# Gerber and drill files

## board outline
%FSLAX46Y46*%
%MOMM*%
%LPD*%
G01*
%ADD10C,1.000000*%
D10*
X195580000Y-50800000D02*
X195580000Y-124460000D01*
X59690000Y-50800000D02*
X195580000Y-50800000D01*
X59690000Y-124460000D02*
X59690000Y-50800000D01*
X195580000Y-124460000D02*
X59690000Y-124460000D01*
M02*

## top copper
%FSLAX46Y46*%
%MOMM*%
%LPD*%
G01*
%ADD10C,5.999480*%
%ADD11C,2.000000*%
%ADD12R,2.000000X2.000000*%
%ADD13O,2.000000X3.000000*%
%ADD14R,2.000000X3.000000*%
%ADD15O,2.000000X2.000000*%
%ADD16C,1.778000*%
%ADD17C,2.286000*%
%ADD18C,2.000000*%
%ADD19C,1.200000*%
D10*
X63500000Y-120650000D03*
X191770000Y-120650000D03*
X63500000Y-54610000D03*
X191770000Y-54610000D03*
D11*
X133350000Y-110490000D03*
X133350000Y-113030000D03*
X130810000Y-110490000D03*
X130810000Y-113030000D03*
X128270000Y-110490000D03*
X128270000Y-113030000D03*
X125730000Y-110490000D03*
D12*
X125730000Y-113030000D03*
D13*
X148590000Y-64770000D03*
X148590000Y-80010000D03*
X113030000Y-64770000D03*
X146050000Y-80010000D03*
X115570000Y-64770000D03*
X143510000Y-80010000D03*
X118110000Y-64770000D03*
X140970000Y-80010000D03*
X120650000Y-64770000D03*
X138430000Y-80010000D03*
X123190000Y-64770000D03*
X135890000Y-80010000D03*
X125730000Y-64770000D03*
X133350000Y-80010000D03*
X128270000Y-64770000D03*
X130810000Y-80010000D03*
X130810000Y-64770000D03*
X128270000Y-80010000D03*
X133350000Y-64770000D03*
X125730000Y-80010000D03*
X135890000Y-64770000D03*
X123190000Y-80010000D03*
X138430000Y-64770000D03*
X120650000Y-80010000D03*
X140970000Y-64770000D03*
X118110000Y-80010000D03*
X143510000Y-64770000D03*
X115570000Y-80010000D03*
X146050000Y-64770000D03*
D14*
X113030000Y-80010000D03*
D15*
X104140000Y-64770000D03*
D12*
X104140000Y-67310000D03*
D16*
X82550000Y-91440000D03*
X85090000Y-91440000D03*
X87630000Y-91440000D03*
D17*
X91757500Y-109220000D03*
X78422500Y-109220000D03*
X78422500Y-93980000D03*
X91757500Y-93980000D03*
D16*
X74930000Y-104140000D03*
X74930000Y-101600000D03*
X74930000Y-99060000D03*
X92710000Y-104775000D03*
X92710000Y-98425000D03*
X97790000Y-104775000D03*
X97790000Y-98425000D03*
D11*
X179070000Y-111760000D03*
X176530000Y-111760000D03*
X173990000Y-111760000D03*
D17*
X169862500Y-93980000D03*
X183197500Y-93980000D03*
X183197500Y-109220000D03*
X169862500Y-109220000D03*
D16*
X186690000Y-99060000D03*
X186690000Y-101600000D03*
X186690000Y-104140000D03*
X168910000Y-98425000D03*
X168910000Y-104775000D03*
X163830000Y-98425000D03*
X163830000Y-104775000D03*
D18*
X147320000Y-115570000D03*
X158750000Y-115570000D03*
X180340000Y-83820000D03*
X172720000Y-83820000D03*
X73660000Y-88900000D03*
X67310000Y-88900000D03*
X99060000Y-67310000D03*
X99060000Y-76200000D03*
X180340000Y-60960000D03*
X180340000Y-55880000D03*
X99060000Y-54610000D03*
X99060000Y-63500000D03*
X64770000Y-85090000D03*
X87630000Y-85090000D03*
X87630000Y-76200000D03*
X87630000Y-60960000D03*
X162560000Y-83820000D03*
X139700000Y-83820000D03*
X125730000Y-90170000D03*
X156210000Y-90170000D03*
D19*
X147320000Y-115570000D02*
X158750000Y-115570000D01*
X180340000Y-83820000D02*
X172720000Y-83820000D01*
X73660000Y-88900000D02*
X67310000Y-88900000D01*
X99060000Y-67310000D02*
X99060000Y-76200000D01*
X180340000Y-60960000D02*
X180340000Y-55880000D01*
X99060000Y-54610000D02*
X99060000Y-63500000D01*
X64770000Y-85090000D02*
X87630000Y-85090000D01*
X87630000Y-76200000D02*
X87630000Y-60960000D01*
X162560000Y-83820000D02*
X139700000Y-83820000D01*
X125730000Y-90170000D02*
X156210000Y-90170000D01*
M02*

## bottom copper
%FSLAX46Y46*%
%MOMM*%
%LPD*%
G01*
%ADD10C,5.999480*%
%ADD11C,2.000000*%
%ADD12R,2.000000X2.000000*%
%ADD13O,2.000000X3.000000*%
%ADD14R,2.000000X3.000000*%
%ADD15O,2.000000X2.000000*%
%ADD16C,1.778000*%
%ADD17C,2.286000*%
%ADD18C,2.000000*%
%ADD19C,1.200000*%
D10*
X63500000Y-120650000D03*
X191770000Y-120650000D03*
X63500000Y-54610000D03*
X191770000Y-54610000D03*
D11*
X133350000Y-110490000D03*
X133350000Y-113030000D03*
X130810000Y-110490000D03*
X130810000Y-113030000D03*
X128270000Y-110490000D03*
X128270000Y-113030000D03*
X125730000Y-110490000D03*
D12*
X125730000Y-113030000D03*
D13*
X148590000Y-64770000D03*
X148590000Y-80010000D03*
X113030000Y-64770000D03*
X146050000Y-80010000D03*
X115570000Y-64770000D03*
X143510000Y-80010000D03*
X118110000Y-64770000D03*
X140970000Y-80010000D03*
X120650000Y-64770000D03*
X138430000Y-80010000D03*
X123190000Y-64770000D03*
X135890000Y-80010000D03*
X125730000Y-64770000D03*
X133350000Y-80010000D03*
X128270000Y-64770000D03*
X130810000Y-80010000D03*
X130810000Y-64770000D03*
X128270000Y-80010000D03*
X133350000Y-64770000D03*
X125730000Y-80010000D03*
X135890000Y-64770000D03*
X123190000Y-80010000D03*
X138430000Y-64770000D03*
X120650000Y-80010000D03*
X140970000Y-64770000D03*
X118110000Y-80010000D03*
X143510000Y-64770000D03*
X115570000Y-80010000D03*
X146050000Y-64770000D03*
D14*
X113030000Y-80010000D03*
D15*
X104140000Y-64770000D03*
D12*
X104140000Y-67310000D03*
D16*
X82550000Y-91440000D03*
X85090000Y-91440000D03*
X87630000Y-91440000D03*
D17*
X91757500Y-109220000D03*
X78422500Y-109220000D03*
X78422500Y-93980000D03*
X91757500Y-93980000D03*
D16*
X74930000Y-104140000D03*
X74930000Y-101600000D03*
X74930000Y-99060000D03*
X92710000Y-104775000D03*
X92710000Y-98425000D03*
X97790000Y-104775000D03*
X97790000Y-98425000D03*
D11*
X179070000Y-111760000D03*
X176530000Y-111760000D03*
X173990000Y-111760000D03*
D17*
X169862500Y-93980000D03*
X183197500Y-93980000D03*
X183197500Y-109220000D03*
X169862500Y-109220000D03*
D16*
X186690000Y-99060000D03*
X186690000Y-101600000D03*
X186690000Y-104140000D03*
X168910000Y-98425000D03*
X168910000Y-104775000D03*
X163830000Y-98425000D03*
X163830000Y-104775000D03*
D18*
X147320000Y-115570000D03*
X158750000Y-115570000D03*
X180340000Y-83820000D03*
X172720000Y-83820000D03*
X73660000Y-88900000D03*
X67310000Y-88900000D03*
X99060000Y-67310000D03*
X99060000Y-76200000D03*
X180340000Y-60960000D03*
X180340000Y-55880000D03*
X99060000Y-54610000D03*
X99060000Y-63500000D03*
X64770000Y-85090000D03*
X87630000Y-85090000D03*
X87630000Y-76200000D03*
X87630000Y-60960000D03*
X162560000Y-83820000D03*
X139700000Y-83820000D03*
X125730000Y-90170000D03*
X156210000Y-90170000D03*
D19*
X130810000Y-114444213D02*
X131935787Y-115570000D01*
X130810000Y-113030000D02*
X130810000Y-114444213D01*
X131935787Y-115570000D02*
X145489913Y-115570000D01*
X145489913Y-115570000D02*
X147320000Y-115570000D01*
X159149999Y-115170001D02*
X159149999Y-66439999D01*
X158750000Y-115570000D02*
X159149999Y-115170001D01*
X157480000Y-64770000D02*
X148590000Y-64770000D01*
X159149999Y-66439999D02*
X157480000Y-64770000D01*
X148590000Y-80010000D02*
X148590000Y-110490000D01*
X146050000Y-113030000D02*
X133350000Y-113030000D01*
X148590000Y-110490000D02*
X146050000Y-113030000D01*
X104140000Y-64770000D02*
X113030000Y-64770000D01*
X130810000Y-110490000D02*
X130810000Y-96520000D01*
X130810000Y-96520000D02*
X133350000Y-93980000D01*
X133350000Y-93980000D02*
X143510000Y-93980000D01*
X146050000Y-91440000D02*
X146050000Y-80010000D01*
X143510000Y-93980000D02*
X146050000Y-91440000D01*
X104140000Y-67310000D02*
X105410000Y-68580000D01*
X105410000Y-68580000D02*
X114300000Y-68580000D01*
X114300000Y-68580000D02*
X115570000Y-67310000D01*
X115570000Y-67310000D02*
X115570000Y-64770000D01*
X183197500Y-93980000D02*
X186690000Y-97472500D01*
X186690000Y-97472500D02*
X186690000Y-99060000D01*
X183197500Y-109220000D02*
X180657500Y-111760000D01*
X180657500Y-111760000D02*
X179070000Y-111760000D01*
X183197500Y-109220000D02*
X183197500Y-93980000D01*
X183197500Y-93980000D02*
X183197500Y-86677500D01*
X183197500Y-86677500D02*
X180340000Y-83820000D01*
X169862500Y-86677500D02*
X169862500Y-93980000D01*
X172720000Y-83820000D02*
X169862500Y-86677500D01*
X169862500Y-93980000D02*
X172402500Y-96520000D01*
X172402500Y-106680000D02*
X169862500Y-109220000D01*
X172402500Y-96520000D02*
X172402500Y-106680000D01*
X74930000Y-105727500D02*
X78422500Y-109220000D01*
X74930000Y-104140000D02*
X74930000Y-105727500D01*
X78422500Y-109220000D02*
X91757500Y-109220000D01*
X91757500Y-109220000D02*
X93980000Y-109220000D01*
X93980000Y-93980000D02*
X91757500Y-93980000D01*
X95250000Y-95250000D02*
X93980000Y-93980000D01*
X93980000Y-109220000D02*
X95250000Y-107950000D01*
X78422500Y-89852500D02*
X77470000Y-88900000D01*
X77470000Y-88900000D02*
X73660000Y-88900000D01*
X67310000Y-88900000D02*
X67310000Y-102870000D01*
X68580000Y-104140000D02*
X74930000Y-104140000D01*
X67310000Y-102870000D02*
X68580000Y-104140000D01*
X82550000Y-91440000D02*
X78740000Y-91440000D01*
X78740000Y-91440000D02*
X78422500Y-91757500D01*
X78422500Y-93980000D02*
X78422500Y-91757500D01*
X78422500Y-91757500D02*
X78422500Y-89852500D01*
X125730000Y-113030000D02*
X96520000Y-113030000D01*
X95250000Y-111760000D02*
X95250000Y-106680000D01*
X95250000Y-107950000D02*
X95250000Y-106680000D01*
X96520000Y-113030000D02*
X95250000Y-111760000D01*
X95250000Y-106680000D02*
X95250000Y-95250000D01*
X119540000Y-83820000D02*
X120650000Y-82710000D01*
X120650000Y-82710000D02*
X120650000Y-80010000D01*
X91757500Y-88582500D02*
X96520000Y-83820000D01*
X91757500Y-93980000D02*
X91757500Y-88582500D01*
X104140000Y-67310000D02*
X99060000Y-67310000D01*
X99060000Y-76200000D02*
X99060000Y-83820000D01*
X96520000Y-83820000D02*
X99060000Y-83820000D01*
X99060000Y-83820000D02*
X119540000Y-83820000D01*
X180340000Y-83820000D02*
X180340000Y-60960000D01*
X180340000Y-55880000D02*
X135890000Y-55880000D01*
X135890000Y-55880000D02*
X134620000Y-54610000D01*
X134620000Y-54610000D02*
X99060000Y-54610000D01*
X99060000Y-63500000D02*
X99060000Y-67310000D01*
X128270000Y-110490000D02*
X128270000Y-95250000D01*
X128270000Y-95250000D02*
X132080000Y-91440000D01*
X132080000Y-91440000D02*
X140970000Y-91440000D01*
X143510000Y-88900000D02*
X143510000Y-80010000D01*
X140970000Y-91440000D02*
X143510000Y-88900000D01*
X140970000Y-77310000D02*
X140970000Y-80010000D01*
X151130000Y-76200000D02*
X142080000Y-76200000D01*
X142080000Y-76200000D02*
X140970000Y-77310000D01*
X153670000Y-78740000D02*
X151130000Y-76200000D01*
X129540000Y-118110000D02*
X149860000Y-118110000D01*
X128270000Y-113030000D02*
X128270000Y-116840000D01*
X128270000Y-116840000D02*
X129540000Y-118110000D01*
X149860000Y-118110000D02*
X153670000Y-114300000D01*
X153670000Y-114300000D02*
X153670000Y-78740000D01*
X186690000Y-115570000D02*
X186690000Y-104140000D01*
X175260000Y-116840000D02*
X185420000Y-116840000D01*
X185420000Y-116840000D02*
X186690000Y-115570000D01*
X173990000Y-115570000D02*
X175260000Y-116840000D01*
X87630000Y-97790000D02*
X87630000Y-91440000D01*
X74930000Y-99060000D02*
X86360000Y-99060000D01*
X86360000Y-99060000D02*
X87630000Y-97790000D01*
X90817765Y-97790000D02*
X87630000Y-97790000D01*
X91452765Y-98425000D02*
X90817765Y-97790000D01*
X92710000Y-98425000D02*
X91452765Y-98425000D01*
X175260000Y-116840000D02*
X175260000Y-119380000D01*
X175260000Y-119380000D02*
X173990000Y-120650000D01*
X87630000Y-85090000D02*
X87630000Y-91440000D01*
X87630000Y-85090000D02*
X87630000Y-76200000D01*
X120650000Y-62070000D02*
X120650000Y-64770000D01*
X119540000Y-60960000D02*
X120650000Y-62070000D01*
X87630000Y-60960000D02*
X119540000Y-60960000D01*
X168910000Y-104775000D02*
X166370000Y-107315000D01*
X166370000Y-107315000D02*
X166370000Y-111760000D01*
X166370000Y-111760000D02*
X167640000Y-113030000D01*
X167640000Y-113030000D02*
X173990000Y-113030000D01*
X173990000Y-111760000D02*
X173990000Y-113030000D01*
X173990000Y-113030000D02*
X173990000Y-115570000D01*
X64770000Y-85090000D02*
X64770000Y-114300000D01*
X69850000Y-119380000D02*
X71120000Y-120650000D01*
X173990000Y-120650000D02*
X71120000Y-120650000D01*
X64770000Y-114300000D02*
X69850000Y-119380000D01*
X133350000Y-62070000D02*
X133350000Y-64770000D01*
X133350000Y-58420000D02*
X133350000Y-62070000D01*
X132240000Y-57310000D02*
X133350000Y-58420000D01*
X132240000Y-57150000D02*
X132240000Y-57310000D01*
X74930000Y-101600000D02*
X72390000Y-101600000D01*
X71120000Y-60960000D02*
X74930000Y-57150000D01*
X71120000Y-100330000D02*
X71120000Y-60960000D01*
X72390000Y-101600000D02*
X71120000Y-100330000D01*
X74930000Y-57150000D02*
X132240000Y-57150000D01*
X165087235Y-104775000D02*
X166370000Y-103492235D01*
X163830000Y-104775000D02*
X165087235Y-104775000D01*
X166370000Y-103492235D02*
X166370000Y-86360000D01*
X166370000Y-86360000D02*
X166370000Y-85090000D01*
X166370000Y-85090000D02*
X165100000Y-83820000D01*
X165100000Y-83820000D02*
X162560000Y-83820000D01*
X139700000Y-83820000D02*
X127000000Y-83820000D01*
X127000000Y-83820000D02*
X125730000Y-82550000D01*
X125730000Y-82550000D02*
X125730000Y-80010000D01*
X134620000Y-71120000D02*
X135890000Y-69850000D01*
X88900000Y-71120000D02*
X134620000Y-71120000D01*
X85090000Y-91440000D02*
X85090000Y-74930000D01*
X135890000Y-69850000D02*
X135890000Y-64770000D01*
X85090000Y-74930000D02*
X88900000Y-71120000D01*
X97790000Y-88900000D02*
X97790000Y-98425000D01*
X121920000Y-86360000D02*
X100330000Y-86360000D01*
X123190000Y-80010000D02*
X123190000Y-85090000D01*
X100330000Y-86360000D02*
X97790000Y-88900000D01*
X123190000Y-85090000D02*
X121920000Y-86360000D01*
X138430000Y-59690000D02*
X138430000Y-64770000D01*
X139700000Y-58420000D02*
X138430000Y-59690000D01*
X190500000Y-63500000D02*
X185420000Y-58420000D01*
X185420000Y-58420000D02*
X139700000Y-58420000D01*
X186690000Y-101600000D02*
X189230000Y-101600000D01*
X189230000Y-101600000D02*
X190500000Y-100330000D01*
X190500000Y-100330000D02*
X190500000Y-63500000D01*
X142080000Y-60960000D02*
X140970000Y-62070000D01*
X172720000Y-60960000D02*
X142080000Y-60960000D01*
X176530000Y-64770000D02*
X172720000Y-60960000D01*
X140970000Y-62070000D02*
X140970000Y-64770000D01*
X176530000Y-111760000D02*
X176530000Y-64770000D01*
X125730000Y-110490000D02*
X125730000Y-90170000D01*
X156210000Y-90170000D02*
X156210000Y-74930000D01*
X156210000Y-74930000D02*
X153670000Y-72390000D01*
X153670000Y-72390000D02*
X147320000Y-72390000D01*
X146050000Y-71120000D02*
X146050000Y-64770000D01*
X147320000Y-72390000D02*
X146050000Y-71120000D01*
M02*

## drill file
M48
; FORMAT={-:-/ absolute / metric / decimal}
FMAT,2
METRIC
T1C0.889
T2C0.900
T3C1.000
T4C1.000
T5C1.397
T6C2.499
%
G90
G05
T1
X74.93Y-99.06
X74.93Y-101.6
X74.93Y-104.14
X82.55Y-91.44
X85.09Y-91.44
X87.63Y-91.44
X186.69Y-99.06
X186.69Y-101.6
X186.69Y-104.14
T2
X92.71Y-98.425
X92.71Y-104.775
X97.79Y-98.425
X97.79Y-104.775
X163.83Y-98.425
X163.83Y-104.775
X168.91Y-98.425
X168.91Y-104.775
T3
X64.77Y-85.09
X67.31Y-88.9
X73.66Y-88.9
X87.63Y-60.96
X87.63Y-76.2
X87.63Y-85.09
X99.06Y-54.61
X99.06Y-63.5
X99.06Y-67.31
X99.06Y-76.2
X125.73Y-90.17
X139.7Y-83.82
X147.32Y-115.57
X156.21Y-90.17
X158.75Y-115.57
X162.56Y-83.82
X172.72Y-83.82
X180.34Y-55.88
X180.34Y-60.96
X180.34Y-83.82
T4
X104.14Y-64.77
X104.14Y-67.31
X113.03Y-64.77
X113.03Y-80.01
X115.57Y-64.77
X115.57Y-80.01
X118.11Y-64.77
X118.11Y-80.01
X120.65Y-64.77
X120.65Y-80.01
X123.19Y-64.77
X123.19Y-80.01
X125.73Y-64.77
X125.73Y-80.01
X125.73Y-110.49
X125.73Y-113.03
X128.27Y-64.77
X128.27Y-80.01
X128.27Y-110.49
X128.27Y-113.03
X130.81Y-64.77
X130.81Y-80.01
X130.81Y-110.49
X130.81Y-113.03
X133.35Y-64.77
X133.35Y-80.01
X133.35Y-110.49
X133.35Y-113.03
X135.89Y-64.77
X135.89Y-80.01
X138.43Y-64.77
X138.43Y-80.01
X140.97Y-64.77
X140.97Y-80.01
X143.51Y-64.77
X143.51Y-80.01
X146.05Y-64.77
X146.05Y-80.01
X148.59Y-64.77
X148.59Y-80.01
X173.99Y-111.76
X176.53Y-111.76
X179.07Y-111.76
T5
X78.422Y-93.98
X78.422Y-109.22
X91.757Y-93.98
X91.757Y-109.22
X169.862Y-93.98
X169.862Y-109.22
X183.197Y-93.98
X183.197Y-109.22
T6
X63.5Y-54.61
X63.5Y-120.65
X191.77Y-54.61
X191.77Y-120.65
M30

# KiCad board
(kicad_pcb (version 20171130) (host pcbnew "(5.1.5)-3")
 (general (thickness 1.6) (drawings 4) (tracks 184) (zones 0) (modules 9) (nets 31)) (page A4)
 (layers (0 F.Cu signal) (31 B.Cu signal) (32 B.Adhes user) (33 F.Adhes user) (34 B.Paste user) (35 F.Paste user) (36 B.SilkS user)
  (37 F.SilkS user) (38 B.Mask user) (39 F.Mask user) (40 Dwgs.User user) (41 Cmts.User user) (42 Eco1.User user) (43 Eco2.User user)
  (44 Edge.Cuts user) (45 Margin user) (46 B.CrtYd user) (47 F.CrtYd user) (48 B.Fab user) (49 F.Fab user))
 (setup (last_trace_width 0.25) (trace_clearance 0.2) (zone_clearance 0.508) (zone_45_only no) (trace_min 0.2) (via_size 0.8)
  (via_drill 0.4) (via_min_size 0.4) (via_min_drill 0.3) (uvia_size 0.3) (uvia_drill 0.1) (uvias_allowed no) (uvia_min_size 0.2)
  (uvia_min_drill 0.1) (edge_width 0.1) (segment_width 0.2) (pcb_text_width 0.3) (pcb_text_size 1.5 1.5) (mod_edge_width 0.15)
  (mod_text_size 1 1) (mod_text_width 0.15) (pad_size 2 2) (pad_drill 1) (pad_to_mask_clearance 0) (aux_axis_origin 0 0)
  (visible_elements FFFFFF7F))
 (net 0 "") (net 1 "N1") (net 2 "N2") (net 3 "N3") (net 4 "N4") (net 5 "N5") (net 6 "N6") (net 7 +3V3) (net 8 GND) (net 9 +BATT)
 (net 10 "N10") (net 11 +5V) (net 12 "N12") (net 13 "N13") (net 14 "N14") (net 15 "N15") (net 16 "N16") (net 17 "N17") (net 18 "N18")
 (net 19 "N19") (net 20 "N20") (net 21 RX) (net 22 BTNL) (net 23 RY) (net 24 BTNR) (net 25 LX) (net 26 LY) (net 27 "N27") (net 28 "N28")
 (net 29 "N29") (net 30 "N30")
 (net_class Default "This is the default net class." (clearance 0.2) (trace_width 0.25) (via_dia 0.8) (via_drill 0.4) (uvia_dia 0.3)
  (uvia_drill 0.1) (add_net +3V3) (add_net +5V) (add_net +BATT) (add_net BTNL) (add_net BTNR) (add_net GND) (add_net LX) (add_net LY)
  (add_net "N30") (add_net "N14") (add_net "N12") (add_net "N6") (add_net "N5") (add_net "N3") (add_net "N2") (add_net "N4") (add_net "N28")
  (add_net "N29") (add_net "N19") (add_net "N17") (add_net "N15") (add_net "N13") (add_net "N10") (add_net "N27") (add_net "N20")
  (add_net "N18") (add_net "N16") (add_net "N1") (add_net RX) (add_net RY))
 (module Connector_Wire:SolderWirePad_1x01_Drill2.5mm (layer F.Cu) (at 63.5 120.65)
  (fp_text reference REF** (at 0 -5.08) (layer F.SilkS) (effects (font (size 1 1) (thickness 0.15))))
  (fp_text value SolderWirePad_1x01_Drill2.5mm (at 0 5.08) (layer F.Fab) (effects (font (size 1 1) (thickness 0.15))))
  (pad 1 thru_hole circle (at 0 0) (size 5.99948 5.99948) (drill 2.49936) (layers *.Cu *.Mask)))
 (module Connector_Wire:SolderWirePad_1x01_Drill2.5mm (layer F.Cu) (at 191.77 120.65)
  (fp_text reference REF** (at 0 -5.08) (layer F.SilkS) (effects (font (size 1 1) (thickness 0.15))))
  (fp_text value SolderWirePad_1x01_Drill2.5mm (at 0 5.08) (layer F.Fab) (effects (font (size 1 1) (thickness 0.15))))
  (pad 1 thru_hole circle (at 0 0) (size 5.99948 5.99948) (drill 2.49936) (layers *.Cu *.Mask)))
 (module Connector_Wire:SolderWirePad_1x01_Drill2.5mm (layer F.Cu) (at 63.5 54.61)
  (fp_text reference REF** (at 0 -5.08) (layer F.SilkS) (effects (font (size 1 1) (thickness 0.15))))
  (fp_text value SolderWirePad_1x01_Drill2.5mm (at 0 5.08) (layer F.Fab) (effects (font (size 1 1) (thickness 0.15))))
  (pad 1 thru_hole circle (at 0 0) (size 5.99948 5.99948) (drill 2.49936) (layers *.Cu *.Mask)))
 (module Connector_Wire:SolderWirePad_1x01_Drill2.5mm (layer F.Cu) (at 191.77 54.61)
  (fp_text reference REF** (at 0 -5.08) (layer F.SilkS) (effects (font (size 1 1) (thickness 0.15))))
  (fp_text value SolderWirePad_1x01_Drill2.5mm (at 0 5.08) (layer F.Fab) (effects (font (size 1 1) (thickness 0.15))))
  (pad 1 thru_hole circle (at 0 0) (size 5.99948 5.99948) (drill 2.49936) (layers *.Cu *.Mask)))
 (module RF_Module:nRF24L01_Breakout (layer F.Cu) (at 125.73 113.03 90)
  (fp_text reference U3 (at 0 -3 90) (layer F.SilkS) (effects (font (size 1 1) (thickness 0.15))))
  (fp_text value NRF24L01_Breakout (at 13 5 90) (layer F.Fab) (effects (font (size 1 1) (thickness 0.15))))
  (pad 8 thru_hole circle (at 2.54 7.62 90) (size 2 2) (drill 1) (layers *.Cu *.Mask) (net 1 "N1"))
  (pad 7 thru_hole circle (at 0 7.62 90) (size 2 2) (drill 1) (layers *.Cu *.Mask) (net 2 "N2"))
  (pad 6 thru_hole circle (at 2.54 5.08 90) (size 2 2) (drill 1) (layers *.Cu *.Mask) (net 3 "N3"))
  (pad 5 thru_hole circle (at 0 5.08 90) (size 2 2) (drill 1) (layers *.Cu *.Mask) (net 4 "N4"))
  (pad 4 thru_hole circle (at 2.54 2.54 90) (size 2 2) (drill 1) (layers *.Cu *.Mask) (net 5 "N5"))
  (pad 3 thru_hole circle (at 0 2.54 90) (size 2 2) (drill 1) (layers *.Cu *.Mask) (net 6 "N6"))
  (pad 2 thru_hole circle (at 2.54 0 90) (size 2 2) (drill 1) (layers *.Cu *.Mask) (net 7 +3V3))
  (pad 1 thru_hole rect (at 0 0 90) (size 2 2) (drill 1) (layers *.Cu *.Mask) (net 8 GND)))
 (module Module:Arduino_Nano (layer F.Cu) (at 113.03 80.01 90)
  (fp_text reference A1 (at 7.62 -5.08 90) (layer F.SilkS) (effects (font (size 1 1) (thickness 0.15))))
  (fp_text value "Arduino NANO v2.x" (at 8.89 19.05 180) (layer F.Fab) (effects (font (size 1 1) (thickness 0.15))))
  (pad 16 thru_hole oval (at 15.24 35.56 90) (size 3 2) (drill 1) (layers *.Cu *.Mask) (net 4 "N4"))
  (pad 15 thru_hole oval (at 0 35.56 90) (size 3 2) (drill 1) (layers *.Cu *.Mask) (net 2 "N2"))
  (pad 30 thru_hole oval (at 15.24 0 90) (size 3 2) (drill 1) (layers *.Cu *.Mask) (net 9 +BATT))
  (pad 14 thru_hole oval (at 0 33.02 90) (size 3 2) (drill 1) (layers *.Cu *.Mask) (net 3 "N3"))
  (pad 29 thru_hole oval (at 15.24 2.54 90) (size 3 2) (drill 1) (layers *.Cu *.Mask) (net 8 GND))
  (pad 13 thru_hole oval (at 0 30.48 90) (size 3 2) (drill 1) (layers *.Cu *.Mask) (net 5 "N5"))
  (pad 28 thru_hole oval (at 15.24 5.08 90) (size 3 2) (drill 1) (layers *.Cu *.Mask) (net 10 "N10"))
  (pad 12 thru_hole oval (at 0 27.94 90) (size 3 2) (drill 1) (layers *.Cu *.Mask) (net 6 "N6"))
  (pad 27 thru_hole oval (at 15.24 7.62 90) (size 3 2) (drill 1) (layers *.Cu *.Mask) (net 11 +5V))
  (pad 11 thru_hole oval (at 0 25.4 90) (size 3 2) (drill 1) (layers *.Cu *.Mask) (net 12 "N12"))
  (pad 26 thru_hole oval (at 15.24 10.16 90) (size 3 2) (drill 1) (layers *.Cu *.Mask) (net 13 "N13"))
  (pad 10 thru_hole oval (at 0 22.86 90) (size 3 2) (drill 1) (layers *.Cu *.Mask) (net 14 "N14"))
  (pad 25 thru_hole oval (at 15.24 12.7 90) (size 3 2) (drill 1) (layers *.Cu *.Mask) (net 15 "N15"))
  (pad 9 thru_hole oval (at 0 20.32 90) (size 3 2) (drill 1) (layers *.Cu *.Mask) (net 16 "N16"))
  (pad 24 thru_hole oval (at 15.24 15.24 90) (size 3 2) (drill 1) (layers *.Cu *.Mask) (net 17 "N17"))
  (pad 8 thru_hole oval (at 0 17.78 90) (size 3 2) (drill 1) (layers *.Cu *.Mask) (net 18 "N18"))
  (pad 23 thru_hole oval (at 15.24 17.78 90) (size 3 2) (drill 1) (layers *.Cu *.Mask) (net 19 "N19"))
  (pad 7 thru_hole oval (at 0 15.24 90) (size 3 2) (drill 1) (layers *.Cu *.Mask) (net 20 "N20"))
  (pad 22 thru_hole oval (at 15.24 20.32 90) (size 3 2) (drill 1) (layers *.Cu *.Mask) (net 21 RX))
  (pad 6 thru_hole oval (at 0 12.7 90) (size 3 2) (drill 1) (layers *.Cu *.Mask) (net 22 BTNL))
  (pad 21 thru_hole oval (at 15.24 22.86 90) (size 3 2) (drill 1) (layers *.Cu *.Mask) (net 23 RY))
  (pad 5 thru_hole oval (at 0 10.16 90) (size 3 2) (drill 1) (layers *.Cu *.Mask) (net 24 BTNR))
  (pad 20 thru_hole oval (at 15.24 25.4 90) (size 3 2) (drill 1) (layers *.Cu *.Mask) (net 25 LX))
  (pad 4 thru_hole oval (at 0 7.62 90) (size 3 2) (drill 1) (layers *.Cu *.Mask) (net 8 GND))
  (pad 19 thru_hole oval (at 15.24 27.94 90) (size 3 2) (drill 1) (layers *.Cu *.Mask) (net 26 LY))
  (pad 3 thru_hole oval (at 0 5.08 90) (size 3 2) (drill 1) (layers *.Cu *.Mask) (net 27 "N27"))
  (pad 18 thru_hole oval (at 15.24 30.48 90) (size 3 2) (drill 1) (layers *.Cu *.Mask) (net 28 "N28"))
  (pad 2 thru_hole oval (at 0 2.54 90) (size 3 2) (drill 1) (layers *.Cu *.Mask) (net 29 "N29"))
  (pad 17 thru_hole oval (at 15.24 33.02 90) (size 3 2) (drill 1) (layers *.Cu *.Mask) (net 7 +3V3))
  (pad 1 thru_hole rect (at 0 0 90) (size 3 2) (drill 1) (layers *.Cu *.Mask) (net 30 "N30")))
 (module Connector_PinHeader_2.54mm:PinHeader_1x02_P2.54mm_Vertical (layer F.Cu) (at 104.14 67.31 180)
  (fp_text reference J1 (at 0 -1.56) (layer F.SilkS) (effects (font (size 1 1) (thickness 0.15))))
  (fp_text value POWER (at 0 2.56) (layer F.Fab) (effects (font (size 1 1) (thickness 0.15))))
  (pad 2 thru_hole oval (at 0 2.54 180) (size 2 2) (drill 1) (layers *.Cu *.Mask) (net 9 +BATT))
  (pad 1 thru_hole rect (at 0 0 180) (size 2 2) (drill 1) (layers *.Cu *.Mask) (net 8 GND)))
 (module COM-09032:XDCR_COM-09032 (layer F.Cu) (at 85.09 101.6 270)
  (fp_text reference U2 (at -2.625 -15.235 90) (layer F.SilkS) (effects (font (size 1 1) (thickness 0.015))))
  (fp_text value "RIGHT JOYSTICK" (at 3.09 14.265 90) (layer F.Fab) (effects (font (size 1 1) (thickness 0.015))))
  (pad V3 thru_hole circle (at -10.16 2.54 270) (size 1.778 1.778) (drill 0.889) (layers *.Cu *.Mask) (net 8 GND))
  (pad V2 thru_hole circle (at -10.16 0 270) (size 1.778 1.778) (drill 0.889) (layers *.Cu *.Mask) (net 23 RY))
  (pad V1 thru_hole circle (at -10.16 -2.54 270) (size 1.778 1.778) (drill 0.889) (layers *.Cu *.Mask) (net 11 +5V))
  (pad S4 thru_hole circle (at 7.62 -6.6675 270) (size 2.286 2.286) (drill 1.397) (layers *.Cu *.Mask) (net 8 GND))
  (pad S3 thru_hole circle (at 7.62 6.6675 270) (size 2.286 2.286) (drill 1.397) (layers *.Cu *.Mask) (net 8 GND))
  (pad S2 thru_hole circle (at -7.62 6.6675 270) (size 2.286 2.286) (drill 1.397) (layers *.Cu *.Mask) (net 8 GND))
  (pad S1 thru_hole circle (at -7.62 -6.6675 270) (size 2.286 2.286) (drill 1.397) (layers *.Cu *.Mask) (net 8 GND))
  (pad H3 thru_hole circle (at 2.54 10.16 270) (size 1.778 1.778) (drill 0.889) (layers *.Cu *.Mask) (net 8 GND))
  (pad H2 thru_hole circle (at 0 10.16 270) (size 1.778 1.778) (drill 0.889) (layers *.Cu *.Mask) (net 21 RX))
  (pad H1 thru_hole circle (at -2.54 10.16 270) (size 1.778 1.778) (drill 0.889) (layers *.Cu *.Mask) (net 11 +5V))
  (pad B2B thru_hole circle (at 3.175 -7.62 270) (size 1.778 1.778) (drill 0.9) (layers *.Cu *.Mask))
  (pad B2A thru_hole circle (at -3.175 -7.62 270) (size 1.778 1.778) (drill 0.9) (layers *.Cu *.Mask) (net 11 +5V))
  (pad B1B thru_hole circle (at 3.175 -12.7 270) (size 1.778 1.778) (drill 0.9) (layers *.Cu *.Mask))
  (pad B1A thru_hole circle (at -3.175 -12.7 270) (size 1.778 1.778) (drill 0.9) (layers *.Cu *.Mask) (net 24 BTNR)))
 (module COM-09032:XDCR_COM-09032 (layer F.Cu) (at 176.53 101.6 90)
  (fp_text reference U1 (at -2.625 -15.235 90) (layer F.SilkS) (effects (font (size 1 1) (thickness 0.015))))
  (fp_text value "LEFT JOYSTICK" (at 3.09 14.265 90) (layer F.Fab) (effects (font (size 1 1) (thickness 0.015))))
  (pad V3 thru_hole circle (at -10.16 2.54 90) (size 2 2) (drill 1) (layers *.Cu *.Mask) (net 8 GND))
  (pad V2 thru_hole circle (at -10.16 0 90) (size 2 2) (drill 1) (layers *.Cu *.Mask) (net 26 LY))
  (pad V1 thru_hole circle (at -10.16 -2.54 90) (size 2 2) (drill 1) (layers *.Cu *.Mask) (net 11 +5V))
  (pad S4 thru_hole circle (at 7.62 -6.6675 90) (size 2.286 2.286) (drill 1.397) (layers *.Cu *.Mask) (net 8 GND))
  (pad S3 thru_hole circle (at 7.62 6.6675 90) (size 2.286 2.286) (drill 1.397) (layers *.Cu *.Mask) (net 8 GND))
  (pad S2 thru_hole circle (at -7.62 6.6675 90) (size 2.286 2.286) (drill 1.397) (layers *.Cu *.Mask) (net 8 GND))
  (pad S1 thru_hole circle (at -7.62 -6.6675 90) (size 2.286 2.286) (drill 1.397) (layers *.Cu *.Mask) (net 8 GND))
  (pad H3 thru_hole circle (at 2.54 10.16 90) (size 1.778 1.778) (drill 0.889) (layers *.Cu *.Mask) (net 8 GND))
  (pad H2 thru_hole circle (at 0 10.16 90) (size 1.778 1.778) (drill 0.889) (layers *.Cu *.Mask) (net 25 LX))
  (pad H1 thru_hole circle (at -2.54 10.16 90) (size 1.778 1.778) (drill 0.889) (layers *.Cu *.Mask) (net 11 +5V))
  (pad B2B thru_hole circle (at 3.175 -7.62 90) (size 1.778 1.778) (drill 0.9) (layers *.Cu *.Mask))
  (pad B2A thru_hole circle (at -3.175 -7.62 90) (size 1.778 1.778) (drill 0.9) (layers *.Cu *.Mask) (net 11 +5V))
  (pad B1B thru_hole circle (at 3.175 -12.7 90) (size 1.778 1.778) (drill 0.9) (layers *.Cu *.Mask))
  (pad B1A thru_hole circle (at -3.175 -12.7 90) (size 1.778 1.778) (drill 0.9) (layers *.Cu *.Mask) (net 22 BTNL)))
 (gr_line (start 195.58 50.8) (end 195.58 124.46) (layer Edge.Cuts) (width 1))
 (gr_line (start 59.69 50.8) (end 195.58 50.8) (layer Edge.Cuts) (width 1))
 (gr_line (start 59.69 124.46) (end 59.69 50.8) (layer Edge.Cuts) (width 1))
 (gr_line (start 195.58 124.46) (end 59.69 124.46) (layer Edge.Cuts) (width 1))
 (segment (start 130.81 114.444213) (end 131.935787 115.57) (width 1.2) (layer B.Cu) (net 4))
 (segment (start 130.81 113.03) (end 130.81 114.444213) (width 1.2) (layer B.Cu) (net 4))
 (via (at 147.32 115.57) (size 2) (drill 1) (layers F.Cu B.Cu) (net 4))
 (segment (start 131.935787 115.57) (end 145.489913 115.57) (width 1.2) (layer B.Cu) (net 4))
 (segment (start 145.489913 115.57) (end 147.32 115.57) (width 1.2) (layer B.Cu) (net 4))
 (via (at 158.75 115.57) (size 2) (drill 1) (layers F.Cu B.Cu) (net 4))
 (segment (start 147.32 115.57) (end 158.75 115.57) (width 1.2) (layer F.Cu) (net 4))
 (segment (start 159.149999 115.170001) (end 159.149999 66.439999) (width 1.2) (layer B.Cu) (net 4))
 (segment (start 158.75 115.57) (end 159.149999 115.170001) (width 1.2) (layer B.Cu) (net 4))
 (segment (start 157.48 64.77) (end 148.59 64.77) (width 1.2) (layer B.Cu) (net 4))
 (segment (start 159.149999 66.439999) (end 157.48 64.77) (width 1.2) (layer B.Cu) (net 4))
 (segment (start 148.59 80.01) (end 148.59 110.49) (width 1.2) (layer B.Cu) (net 2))
 (segment (start 146.05 113.03) (end 133.35 113.03) (width 1.2) (layer B.Cu) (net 2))
 (segment (start 148.59 110.49) (end 146.05 113.03) (width 1.2) (layer B.Cu) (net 2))
 (segment (start 104.14 64.77) (end 113.03 64.77) (width 1.2) (layer B.Cu) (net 9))
 (segment (start 130.81 110.49) (end 130.81 96.52) (width 1.2) (layer B.Cu) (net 3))
 (segment (start 130.81 96.52) (end 133.35 93.98) (width 1.2) (layer B.Cu) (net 3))
 (segment (start 133.35 93.98) (end 143.51 93.98) (width 1.2) (layer B.Cu) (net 3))
 (segment (start 146.05 91.44) (end 146.05 80.01) (width 1.2) (layer B.Cu) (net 3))
 (segment (start 143.51 93.98) (end 146.05 91.44) (width 1.2) (layer B.Cu) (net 3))
 (segment (start 104.14 67.31) (end 105.41 68.58) (width 1.2) (layer B.Cu) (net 8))
 (segment (start 105.41 68.58) (end 114.3 68.58) (width 1.2) (layer B.Cu) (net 8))
 (segment (start 114.3 68.58) (end 115.57 67.31) (width 1.2) (layer B.Cu) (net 8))
 (segment (start 115.57 67.31) (end 115.57 64.77) (width 1.2) (layer B.Cu) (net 8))
 (segment (start 183.1975 93.98) (end 186.69 97.4725) (width 1.2) (layer B.Cu) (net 8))
 (segment (start 186.69 97.4725) (end 186.69 99.06) (width 1.2) (layer B.Cu) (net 8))
 (segment (start 183.1975 109.22) (end 180.6575 111.76) (width 1.2) (layer B.Cu) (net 8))
 (segment (start 180.6575 111.76) (end 179.07 111.76) (width 1.2) (layer B.Cu) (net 8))
 (segment (start 183.1975 109.22) (end 183.1975 93.98) (width 1.2) (layer B.Cu) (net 8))
 (via (at 180.34 83.82) (size 2) (drill 1) (layers F.Cu B.Cu) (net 8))
 (segment (start 183.1975 93.98) (end 183.1975 86.6775) (width 1.2) (layer B.Cu) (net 8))
 (segment (start 183.1975 86.6775) (end 180.34 83.82) (width 1.2) (layer B.Cu) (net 8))
 (via (at 172.72 83.82) (size 2) (drill 1) (layers F.Cu B.Cu) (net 8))
 (segment (start 180.34 83.82) (end 172.72 83.82) (width 1.2) (layer F.Cu) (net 8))
 (segment (start 169.8625 86.6775) (end 169.8625 93.98) (width 1.2) (layer B.Cu) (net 8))
 (segment (start 172.72 83.82) (end 169.8625 86.6775) (width 1.2) (layer B.Cu) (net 8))
 (segment (start 169.8625 93.98) (end 172.4025 96.52) (width 1.2) (layer B.Cu) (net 8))
 (segment (start 172.4025 106.68) (end 169.8625 109.22) (width 1.2) (layer B.Cu) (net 8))
 (segment (start 172.4025 96.52) (end 172.4025 106.68) (width 1.2) (layer B.Cu) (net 8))
 (segment (start 74.93 105.7275) (end 78.4225 109.22) (width 1.2) (layer B.Cu) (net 8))
 (segment (start 74.93 104.14) (end 74.93 105.7275) (width 1.2) (layer B.Cu) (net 8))
 (segment (start 78.4225 109.22) (end 91.7575 109.22) (width 1.2) (layer B.Cu) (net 8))
 (segment (start 91.7575 109.22) (end 93.98 109.22) (width 1.2) (layer B.Cu) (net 8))
 (segment (start 93.98 93.98) (end 91.7575 93.98) (width 1.2) (layer B.Cu) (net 8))
 (segment (start 95.25 95.25) (end 93.98 93.98) (width 1.2) (layer B.Cu) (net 8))
 (segment (start 93.98 109.22) (end 95.25 107.95) (width 1.2) (layer B.Cu) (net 8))
 (via (at 73.66 88.9) (size 2) (drill 1) (layers F.Cu B.Cu) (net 8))
 (segment (start 78.4225 89.8525) (end 77.47 88.9) (width 1.2) (layer B.Cu) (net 8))
 (segment (start 77.47 88.9) (end 73.66 88.9) (width 1.2) (layer B.Cu) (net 8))
 (via (at 67.31 88.9) (size 2) (drill 1) (layers F.Cu B.Cu) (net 8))
 (segment (start 73.66 88.9) (end 67.31 88.9) (width 1.2) (layer F.Cu) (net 8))
 (segment (start 67.31 88.9) (end 67.31 102.87) (width 1.2) (layer B.Cu) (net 8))
 (segment (start 68.58 104.14) (end 74.93 104.14) (width 1.2) (layer B.Cu) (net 8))
 (segment (start 67.31 102.87) (end 68.58 104.14) (width 1.2) (layer B.Cu) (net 8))
 (segment (start 82.55 91.44) (end 78.74 91.44) (width 1.2) (layer B.Cu) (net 8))
 (segment (start 78.74 91.44) (end 78.4225 91.7575) (width 1.2) (layer B.Cu) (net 8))
 (segment (start 78.4225 93.98) (end 78.4225 91.7575) (width 1.2) (layer B.Cu) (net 8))
 (segment (start 78.4225 91.7575) (end 78.4225 89.8525) (width 1.2) (layer B.Cu) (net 8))
 (segment (start 125.73 113.03) (end 96.52 113.03) (width 1.2) (layer B.Cu) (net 8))
 (segment (start 95.25 111.76) (end 95.25 106.68) (width 1.2) (layer B.Cu) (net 8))
 (segment (start 95.25 107.95) (end 95.25 106.68) (width 1.2) (layer B.Cu) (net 8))
 (segment (start 96.52 113.03) (end 95.25 111.76) (width 1.2) (layer B.Cu) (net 8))
 (segment (start 95.25 106.68) (end 95.25 95.25) (width 1.2) (layer B.Cu) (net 8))
 (segment (start 119.54 83.82) (end 120.65 82.71) (width 1.2) (layer B.Cu) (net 8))
 (segment (start 120.65 82.71) (end 120.65 80.01) (width 1.2) (layer B.Cu) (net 8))
 (segment (start 91.7575 88.5825) (end 96.52 83.82) (width 1.2) (layer B.Cu) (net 8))
 (segment (start 91.7575 93.98) (end 91.7575 88.5825) (width 1.2) (layer B.Cu) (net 8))
 (via (at 99.06 67.31) (size 2) (drill 1) (layers F.Cu B.Cu) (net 8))
 (segment (start 104.14 67.31) (end 99.06 67.31) (width 1.2) (layer B.Cu) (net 8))
 (via (at 99.06 76.2) (size 2) (drill 1) (layers F.Cu B.Cu) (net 8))
 (segment (start 99.06 67.31) (end 99.06 76.2) (width 1.2) (layer F.Cu) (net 8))
 (segment (start 99.06 76.2) (end 99.06 83.82) (width 1.2) (layer B.Cu) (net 8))
 (segment (start 96.52 83.82) (end 99.06 83.82) (width 1.2) (layer B.Cu) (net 8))
 (segment (start 99.06 83.82) (end 119.54 83.82) (width 1.2) (layer B.Cu) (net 8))
 (via (at 180.34 60.96) (size 2) (drill 1) (layers F.Cu B.Cu) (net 8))
 (segment (start 180.34 83.82) (end 180.34 60.96) (width 1.2) (layer B.Cu) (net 8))
 (via (at 180.34 55.88) (size 2) (drill 1) (layers F.Cu B.Cu) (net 8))
 (segment (start 180.34 60.96) (end 180.34 55.88) (width 1.2) (layer F.Cu) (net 8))
 (segment (start 180.34 55.88) (end 135.89 55.88) (width 1.2) (layer B.Cu) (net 8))
 (segment (start 135.89 55.88) (end 134.62 54.61) (width 1.2) (layer B.Cu) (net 8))
 (via (at 99.06 54.61) (size 2) (drill 1) (layers F.Cu B.Cu) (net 8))
 (segment (start 134.62 54.61) (end 99.06 54.61) (width 1.2) (layer B.Cu) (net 8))
 (via (at 99.06 63.5) (size 2) (drill 1) (layers F.Cu B.Cu) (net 8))
 (segment (start 99.06 54.61) (end 99.06 63.5) (width 1.2) (layer F.Cu) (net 8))
 (segment (start 99.06 63.5) (end 99.06 67.31) (width 1.2) (layer B.Cu) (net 8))
 (segment (start 128.27 110.49) (end 128.27 95.25) (width 1.2) (layer B.Cu) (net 5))
 (segment (start 128.27 95.25) (end 132.08 91.44) (width 1.2) (layer B.Cu) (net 5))
 (segment (start 132.08 91.44) (end 140.97 91.44) (width 1.2) (layer B.Cu) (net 5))
 (segment (start 143.51 88.9) (end 143.51 80.01) (width 1.2) (layer B.Cu) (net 5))
 (segment (start 140.97 91.44) (end 143.51 88.9) (width 1.2) (layer B.Cu) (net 5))
 (segment (start 140.97 77.31) (end 140.97 80.01) (width 1.2) (layer B.Cu) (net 6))
 (segment (start 151.13 76.2) (end 142.08 76.2) (width 1.2) (layer B.Cu) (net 6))
 (segment (start 142.08 76.2) (end 140.97 77.31) (width 1.2) (layer B.Cu) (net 6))
 (segment (start 153.67 78.74) (end 151.13 76.2) (width 1.2) (layer B.Cu) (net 6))
 (segment (start 129.54 118.11) (end 149.86 118.11) (width 1.2) (layer B.Cu) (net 6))
 (segment (start 128.27 113.03) (end 128.27 116.84) (width 1.2) (layer B.Cu) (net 6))
 (segment (start 128.27 116.84) (end 129.54 118.11) (width 1.2) (layer B.Cu) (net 6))
 (segment (start 149.86 118.11) (end 153.67 114.3) (width 1.2) (layer B.Cu) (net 6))
 (segment (start 153.67 114.3) (end 153.67 78.74) (width 1.2) (layer B.Cu) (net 6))
 (segment (start 186.69 115.57) (end 186.69 104.14) (width 1.2) (layer B.Cu) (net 11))
 (segment (start 175.26 116.84) (end 185.42 116.84) (width 1.2) (layer B.Cu) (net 11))
 (segment (start 185.42 116.84) (end 186.69 115.57) (width 1.2) (layer B.Cu) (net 11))
 (segment (start 173.99 115.57) (end 175.26 116.84) (width 1.2) (layer B.Cu) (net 11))
 (segment (start 87.63 97.79) (end 87.63 91.44) (width 1.2) (layer B.Cu) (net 11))
 (segment (start 74.93 99.06) (end 86.36 99.06) (width 1.2) (layer B.Cu) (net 11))
 (segment (start 86.36 99.06) (end 87.63 97.79) (width 1.2) (layer B.Cu) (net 11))
 (segment (start 90.817765 97.79) (end 87.63 97.79) (width 1.2) (layer B.Cu) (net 11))
 (segment (start 91.452765 98.425) (end 90.817765 97.79) (width 1.2) (layer B.Cu) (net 11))
 (segment (start 92.71 98.425) (end 91.452765 98.425) (width 1.2) (layer B.Cu) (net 11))
 (segment (start 175.26 116.84) (end 175.26 119.38) (width 1.2) (layer B.Cu) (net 11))
 (segment (start 175.26 119.38) (end 173.99 120.65) (width 1.2) (layer B.Cu) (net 11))
 (via (at 64.77 85.09) (size 2) (drill 1) (layers F.Cu B.Cu) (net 11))
 (via (at 87.63 85.09) (size 2) (drill 1) (layers F.Cu B.Cu) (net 11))
 (segment (start 64.77 85.09) (end 87.63 85.09) (width 1.2) (layer F.Cu) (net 11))
 (segment (start 87.63 85.09) (end 87.63 91.44) (width 1.2) (layer B.Cu) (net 11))
 (via (at 87.63 76.2) (size 2) (drill 1) (layers F.Cu B.Cu) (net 11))
 (segment (start 87.63 85.09) (end 87.63 76.2) (width 1.2) (layer B.Cu) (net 11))
 (via (at 87.63 60.96) (size 2) (drill 1) (layers F.Cu B.Cu) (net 11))
 (segment (start 87.63 76.2) (end 87.63 60.96) (width 1.2) (layer F.Cu) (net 11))
 (segment (start 120.65 62.07) (end 120.65 64.77) (width 1.2) (layer B.Cu) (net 11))
 (segment (start 119.54 60.96) (end 120.65 62.07) (width 1.2) (layer B.Cu) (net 11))
 (segment (start 87.63 60.96) (end 119.54 60.96) (width 1.2) (layer B.Cu) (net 11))
 (segment (start 168.91 104.775) (end 166.37 107.315) (width 1.2) (layer B.Cu) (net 11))
 (segment (start 166.37 107.315) (end 166.37 111.76) (width 1.2) (layer B.Cu) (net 11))
 (segment (start 166.37 111.76) (end 167.64 113.03) (width 1.2) (layer B.Cu) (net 11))
 (segment (start 167.64 113.03) (end 173.99 113.03) (width 1.2) (layer B.Cu) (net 11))
 (segment (start 173.99 111.76) (end 173.99 113.03) (width 1.2) (layer B.Cu) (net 11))
 (segment (start 173.99 113.03) (end 173.99 115.57) (width 1.2) (layer B.Cu) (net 11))
 (segment (start 64.77 85.09) (end 64.77 114.3) (width 1.2) (layer B.Cu) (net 11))
 (segment (start 69.85 119.38) (end 71.12 120.65) (width 1.2) (layer B.Cu) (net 11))
 (segment (start 173.99 120.65) (end 71.12 120.65) (width 1.2) (layer B.Cu) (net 11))
 (segment (start 64.77 114.3) (end 69.85 119.38) (width 1.2) (layer B.Cu) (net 11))
 (segment (start 133.35 62.07) (end 133.35 64.77) (width 1.2) (layer B.Cu) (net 21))
 (segment (start 133.35 58.42) (end 133.35 62.07) (width 1.2) (layer B.Cu) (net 21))
 (segment (start 132.24 57.31) (end 133.35 58.42) (width 1.2) (layer B.Cu) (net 21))
 (segment (start 132.24 57.15) (end 132.24 57.31) (width 1.2) (layer B.Cu) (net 21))
 (segment (start 74.93 101.6) (end 72.39 101.6) (width 1.2) (layer B.Cu) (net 21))
 (segment (start 71.12 60.96) (end 74.93 57.15) (width 1.2) (layer B.Cu) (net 21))
 (segment (start 71.12 100.33) (end 71.12 60.96) (width 1.2) (layer B.Cu) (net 21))
 (segment (start 72.39 101.6) (end 71.12 100.33) (width 1.2) (layer B.Cu) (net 21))
 (segment (start 74.93 57.15) (end 132.24 57.15) (width 1.2) (layer B.Cu) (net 21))
 (segment (start 165.087235 104.775) (end 166.37 103.492235) (width 1.2) (layer B.Cu) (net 22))
 (segment (start 163.83 104.775) (end 165.087235 104.775) (width 1.2) (layer B.Cu) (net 22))
 (segment (start 166.37 103.492235) (end 166.37 86.36) (width 1.2) (layer B.Cu) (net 22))
 (segment (start 166.37 86.36) (end 166.37 85.09) (width 1.2) (layer B.Cu) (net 22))
 (via (at 162.56 83.82) (size 2) (drill 1) (layers F.Cu B.Cu) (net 22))
 (segment (start 166.37 85.09) (end 165.1 83.82) (width 1.2) (layer B.Cu) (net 22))
 (segment (start 165.1 83.82) (end 162.56 83.82) (width 1.2) (layer B.Cu) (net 22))
 (via (at 139.7 83.82) (size 2) (drill 1) (layers F.Cu B.Cu) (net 22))
 (segment (start 162.56 83.82) (end 139.7 83.82) (width 1.2) (layer F.Cu) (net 22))
 (segment (start 139.7 83.82) (end 127 83.82) (width 1.2) (layer B.Cu) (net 22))
 (segment (start 127 83.82) (end 125.73 82.55) (width 1.2) (layer B.Cu) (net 22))
 (segment (start 125.73 82.55) (end 125.73 80.01) (width 1.2) (layer B.Cu) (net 22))
 (segment (start 134.62 71.12) (end 135.89 69.85) (width 1.2) (layer B.Cu) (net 23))
 (segment (start 88.9 71.12) (end 134.62 71.12) (width 1.2) (layer B.Cu) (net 23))
 (segment (start 85.09 91.44) (end 85.09 74.93) (width 1.2) (layer B.Cu) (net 23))
 (segment (start 135.89 69.85) (end 135.89 64.77) (width 1.2) (layer B.Cu) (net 23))
 (segment (start 85.09 74.93) (end 88.9 71.12) (width 1.2) (layer B.Cu) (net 23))
 (segment (start 97.79 88.9) (end 97.79 98.425) (width 1.2) (layer B.Cu) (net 24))
 (segment (start 121.92 86.36) (end 100.33 86.36) (width 1.2) (layer B.Cu) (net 24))
 (segment (start 123.19 80.01) (end 123.19 85.09) (width 1.2) (layer B.Cu) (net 24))
 (segment (start 100.33 86.36) (end 97.79 88.9) (width 1.2) (layer B.Cu) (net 24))
 (segment (start 123.19 85.09) (end 121.92 86.36) (width 1.2) (layer B.Cu) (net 24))
 (segment (start 138.43 59.69) (end 138.43 64.77) (width 1.2) (layer B.Cu) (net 25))
 (segment (start 139.7 58.42) (end 138.43 59.69) (width 1.2) (layer B.Cu) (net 25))
 (segment (start 190.5 63.5) (end 185.42 58.42) (width 1.2) (layer B.Cu) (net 25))
 (segment (start 185.42 58.42) (end 139.7 58.42) (width 1.2) (layer B.Cu) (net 25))
 (segment (start 186.69 101.6) (end 189.23 101.6) (width 1.2) (layer B.Cu) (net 25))
 (segment (start 189.23 101.6) (end 190.5 100.33) (width 1.2) (layer B.Cu) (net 25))
 (segment (start 190.5 100.33) (end 190.5 63.5) (width 1.2) (layer B.Cu) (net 25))
 (segment (start 142.08 60.96) (end 140.97 62.07) (width 1.2) (layer B.Cu) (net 26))
 (segment (start 172.72 60.96) (end 142.08 60.96) (width 1.2) (layer B.Cu) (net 26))
 (segment (start 176.53 64.77) (end 172.72 60.96) (width 1.2) (layer B.Cu) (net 26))
 (segment (start 140.97 62.07) (end 140.97 64.77) (width 1.2) (layer B.Cu) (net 26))
 (segment (start 176.53 111.76) (end 176.53 64.77) (width 1.2) (layer B.Cu) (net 26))
 (via (at 125.73 90.17) (size 2) (drill 1) (layers F.Cu B.Cu) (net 7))
 (segment (start 125.73 110.49) (end 125.73 90.17) (width 1.2) (layer B.Cu) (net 7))
 (via (at 156.21 90.17) (size 2) (drill 1) (layers F.Cu B.Cu) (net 7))
 (segment (start 125.73 90.17) (end 156.21 90.17) (width 1.2) (layer F.Cu) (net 7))
 (segment (start 156.21 90.17) (end 156.21 74.93) (width 1.2) (layer B.Cu) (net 7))
 (segment (start 156.21 74.93) (end 153.67 72.39) (width 1.2) (layer B.Cu) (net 7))
 (segment (start 153.67 72.39) (end 147.32 72.39) (width 1.2) (layer B.Cu) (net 7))
 (segment (start 146.05 71.12) (end 146.05 64.77) (width 1.2) (layer B.Cu) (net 7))
 (segment (start 147.32 72.39) (end 146.05 71.12) (width 1.2) (layer B.Cu) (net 7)))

